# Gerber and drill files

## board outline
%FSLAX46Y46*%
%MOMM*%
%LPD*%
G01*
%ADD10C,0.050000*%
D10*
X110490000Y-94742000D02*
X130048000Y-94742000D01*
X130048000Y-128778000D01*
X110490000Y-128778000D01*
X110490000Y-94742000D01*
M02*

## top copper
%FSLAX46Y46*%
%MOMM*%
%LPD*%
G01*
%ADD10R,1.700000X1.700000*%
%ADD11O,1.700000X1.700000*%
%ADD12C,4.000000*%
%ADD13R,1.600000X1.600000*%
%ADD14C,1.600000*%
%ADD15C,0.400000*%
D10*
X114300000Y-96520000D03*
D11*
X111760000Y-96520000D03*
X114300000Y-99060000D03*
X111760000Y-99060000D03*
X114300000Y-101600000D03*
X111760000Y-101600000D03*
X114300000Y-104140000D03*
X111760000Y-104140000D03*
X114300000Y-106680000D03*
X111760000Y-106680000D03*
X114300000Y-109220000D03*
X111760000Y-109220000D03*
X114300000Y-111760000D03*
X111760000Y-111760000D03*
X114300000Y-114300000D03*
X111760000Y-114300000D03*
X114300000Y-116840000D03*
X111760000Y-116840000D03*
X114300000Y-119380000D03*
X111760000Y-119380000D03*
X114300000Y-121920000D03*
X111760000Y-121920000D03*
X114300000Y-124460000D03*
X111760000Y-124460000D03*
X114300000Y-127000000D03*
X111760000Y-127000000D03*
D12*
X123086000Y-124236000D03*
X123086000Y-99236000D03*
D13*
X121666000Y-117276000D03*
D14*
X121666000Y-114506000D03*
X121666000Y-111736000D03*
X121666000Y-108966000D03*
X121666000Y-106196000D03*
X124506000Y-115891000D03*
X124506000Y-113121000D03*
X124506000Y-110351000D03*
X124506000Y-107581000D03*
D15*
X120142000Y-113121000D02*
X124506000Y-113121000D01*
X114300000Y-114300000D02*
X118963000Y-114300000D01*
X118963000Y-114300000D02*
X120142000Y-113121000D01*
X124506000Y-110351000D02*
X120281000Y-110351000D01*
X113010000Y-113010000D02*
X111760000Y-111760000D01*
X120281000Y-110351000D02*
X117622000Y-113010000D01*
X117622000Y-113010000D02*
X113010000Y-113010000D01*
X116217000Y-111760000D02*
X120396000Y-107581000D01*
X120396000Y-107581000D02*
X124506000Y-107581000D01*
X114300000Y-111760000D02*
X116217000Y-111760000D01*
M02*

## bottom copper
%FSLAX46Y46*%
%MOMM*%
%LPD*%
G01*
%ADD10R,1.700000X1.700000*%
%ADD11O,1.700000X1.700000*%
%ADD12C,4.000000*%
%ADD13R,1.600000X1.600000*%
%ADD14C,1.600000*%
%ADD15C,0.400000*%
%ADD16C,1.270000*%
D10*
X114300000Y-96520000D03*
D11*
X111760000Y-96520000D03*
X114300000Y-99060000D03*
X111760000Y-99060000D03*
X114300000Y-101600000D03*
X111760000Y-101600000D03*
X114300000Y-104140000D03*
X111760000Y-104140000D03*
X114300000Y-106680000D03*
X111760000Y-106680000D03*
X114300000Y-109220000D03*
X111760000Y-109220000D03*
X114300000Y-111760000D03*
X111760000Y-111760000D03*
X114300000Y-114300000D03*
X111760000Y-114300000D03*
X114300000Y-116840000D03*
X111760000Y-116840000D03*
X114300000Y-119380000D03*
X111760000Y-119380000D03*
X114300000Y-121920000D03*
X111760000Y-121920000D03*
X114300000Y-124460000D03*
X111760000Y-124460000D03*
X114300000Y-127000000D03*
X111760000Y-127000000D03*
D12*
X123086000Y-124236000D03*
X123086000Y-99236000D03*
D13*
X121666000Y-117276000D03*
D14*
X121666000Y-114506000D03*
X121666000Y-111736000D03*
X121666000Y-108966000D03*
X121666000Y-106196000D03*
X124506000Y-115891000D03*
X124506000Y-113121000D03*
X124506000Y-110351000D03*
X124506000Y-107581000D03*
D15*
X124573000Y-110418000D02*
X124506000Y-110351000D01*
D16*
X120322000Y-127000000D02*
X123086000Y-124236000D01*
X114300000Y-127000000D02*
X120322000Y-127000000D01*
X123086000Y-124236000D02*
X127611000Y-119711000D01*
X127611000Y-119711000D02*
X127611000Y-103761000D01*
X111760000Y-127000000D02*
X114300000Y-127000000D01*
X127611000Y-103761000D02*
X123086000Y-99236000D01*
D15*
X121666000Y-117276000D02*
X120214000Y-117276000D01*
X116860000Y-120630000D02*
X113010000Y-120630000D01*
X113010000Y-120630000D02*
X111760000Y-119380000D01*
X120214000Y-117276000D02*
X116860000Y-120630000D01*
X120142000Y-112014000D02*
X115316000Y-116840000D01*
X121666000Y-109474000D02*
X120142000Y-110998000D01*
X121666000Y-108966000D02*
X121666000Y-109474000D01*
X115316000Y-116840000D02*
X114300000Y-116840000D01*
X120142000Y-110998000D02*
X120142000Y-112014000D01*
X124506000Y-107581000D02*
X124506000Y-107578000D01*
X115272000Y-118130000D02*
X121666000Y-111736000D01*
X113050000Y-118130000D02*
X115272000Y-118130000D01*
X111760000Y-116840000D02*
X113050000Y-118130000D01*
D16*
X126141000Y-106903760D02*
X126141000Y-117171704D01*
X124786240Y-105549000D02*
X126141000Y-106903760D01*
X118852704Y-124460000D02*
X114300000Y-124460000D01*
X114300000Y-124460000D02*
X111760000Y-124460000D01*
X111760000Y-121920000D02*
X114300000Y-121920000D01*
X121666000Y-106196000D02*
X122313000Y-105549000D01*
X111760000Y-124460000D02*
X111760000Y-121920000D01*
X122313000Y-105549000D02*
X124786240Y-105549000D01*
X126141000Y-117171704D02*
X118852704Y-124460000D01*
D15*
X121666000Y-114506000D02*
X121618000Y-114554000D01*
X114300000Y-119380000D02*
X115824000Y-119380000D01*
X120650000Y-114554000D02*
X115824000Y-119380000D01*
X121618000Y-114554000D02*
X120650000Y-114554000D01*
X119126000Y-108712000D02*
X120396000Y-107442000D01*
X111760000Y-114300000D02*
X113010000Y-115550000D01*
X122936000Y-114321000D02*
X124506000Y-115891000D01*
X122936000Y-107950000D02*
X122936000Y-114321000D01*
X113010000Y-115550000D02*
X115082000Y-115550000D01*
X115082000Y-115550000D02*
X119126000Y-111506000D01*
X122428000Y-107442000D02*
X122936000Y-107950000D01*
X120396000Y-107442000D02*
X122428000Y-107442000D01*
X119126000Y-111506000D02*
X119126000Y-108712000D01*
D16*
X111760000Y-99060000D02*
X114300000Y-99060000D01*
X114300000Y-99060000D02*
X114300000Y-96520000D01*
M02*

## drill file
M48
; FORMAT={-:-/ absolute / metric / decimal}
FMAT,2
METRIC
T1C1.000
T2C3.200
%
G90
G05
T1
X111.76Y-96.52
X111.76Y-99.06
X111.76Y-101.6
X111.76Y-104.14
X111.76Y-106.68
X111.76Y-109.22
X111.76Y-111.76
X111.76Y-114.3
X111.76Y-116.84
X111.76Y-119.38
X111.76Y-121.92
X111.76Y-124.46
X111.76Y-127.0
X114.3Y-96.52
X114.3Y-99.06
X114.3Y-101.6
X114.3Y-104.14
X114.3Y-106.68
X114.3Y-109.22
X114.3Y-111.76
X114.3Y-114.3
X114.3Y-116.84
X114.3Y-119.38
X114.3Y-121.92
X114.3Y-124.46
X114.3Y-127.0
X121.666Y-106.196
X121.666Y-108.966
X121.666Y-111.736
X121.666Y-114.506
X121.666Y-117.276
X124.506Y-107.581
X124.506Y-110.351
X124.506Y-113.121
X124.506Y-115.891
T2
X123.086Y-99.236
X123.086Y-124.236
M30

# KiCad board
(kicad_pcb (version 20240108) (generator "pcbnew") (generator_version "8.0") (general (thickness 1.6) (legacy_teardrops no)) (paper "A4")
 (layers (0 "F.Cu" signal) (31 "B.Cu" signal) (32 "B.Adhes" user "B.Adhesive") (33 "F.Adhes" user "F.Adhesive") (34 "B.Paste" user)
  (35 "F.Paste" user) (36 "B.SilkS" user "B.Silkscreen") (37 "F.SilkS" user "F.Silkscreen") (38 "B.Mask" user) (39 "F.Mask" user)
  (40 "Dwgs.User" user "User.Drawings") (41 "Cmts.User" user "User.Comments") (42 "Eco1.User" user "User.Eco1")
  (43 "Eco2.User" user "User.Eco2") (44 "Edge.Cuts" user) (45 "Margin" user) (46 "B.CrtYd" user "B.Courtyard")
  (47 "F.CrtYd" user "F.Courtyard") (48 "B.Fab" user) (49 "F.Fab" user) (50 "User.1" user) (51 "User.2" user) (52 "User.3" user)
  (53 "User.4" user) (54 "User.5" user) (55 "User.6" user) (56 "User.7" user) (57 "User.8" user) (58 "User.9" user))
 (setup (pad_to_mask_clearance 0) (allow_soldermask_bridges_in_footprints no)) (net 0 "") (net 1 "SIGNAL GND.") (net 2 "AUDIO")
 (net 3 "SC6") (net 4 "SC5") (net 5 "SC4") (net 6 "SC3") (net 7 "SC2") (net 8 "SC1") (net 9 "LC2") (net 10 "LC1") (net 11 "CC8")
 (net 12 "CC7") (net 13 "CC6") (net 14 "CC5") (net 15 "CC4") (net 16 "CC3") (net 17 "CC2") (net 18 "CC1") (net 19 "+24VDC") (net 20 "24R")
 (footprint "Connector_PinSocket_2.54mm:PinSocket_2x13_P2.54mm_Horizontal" (layer "F.Cu") (at 114.3 96.52)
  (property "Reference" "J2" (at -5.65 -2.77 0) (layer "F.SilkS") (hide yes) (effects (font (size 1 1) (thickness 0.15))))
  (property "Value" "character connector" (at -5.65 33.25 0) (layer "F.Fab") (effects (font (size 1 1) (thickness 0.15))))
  (pad "1" thru_hole rect (at 0 0) (size 1.7 1.7) (drill 1) (layers "*.Cu" "*.Mask") (remove_unused_layers no) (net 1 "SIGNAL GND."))
  (pad "2" thru_hole oval (at -2.54 0) (size 1.7 1.7) (drill 1) (layers "*.Cu" "*.Mask") (remove_unused_layers no) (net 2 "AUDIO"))
  (pad "3" thru_hole oval (at 0 2.54) (size 1.7 1.7) (drill 1) (layers "*.Cu" "*.Mask") (remove_unused_layers no) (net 1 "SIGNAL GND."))
  (pad "4" thru_hole oval (at -2.54 2.54) (size 1.7 1.7) (drill 1) (layers "*.Cu" "*.Mask") (remove_unused_layers no) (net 1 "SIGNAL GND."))
  (pad "5" thru_hole oval (at 0 5.08) (size 1.7 1.7) (drill 1) (layers "*.Cu" "*.Mask") (remove_unused_layers no) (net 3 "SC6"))
  (pad "6" thru_hole oval (at -2.54 5.08) (size 1.7 1.7) (drill 1) (layers "*.Cu" "*.Mask") (remove_unused_layers no) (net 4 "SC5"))
  (pad "7" thru_hole oval (at 0 7.62) (size 1.7 1.7) (drill 1) (layers "*.Cu" "*.Mask") (remove_unused_layers no) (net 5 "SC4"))
  (pad "8" thru_hole oval (at -2.54 7.62) (size 1.7 1.7) (drill 1) (layers "*.Cu" "*.Mask") (remove_unused_layers no) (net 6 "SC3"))
  (pad "9" thru_hole oval (at 0 10.16) (size 1.7 1.7) (drill 1) (layers "*.Cu" "*.Mask") (remove_unused_layers no) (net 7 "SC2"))
  (pad "10" thru_hole oval (at -2.54 10.16) (size 1.7 1.7) (drill 1) (layers "*.Cu" "*.Mask") (remove_unused_layers no) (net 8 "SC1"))
  (pad "11" thru_hole oval (at 0 12.7) (size 1.7 1.7) (drill 1) (layers "*.Cu" "*.Mask") (remove_unused_layers no) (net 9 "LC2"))
  (pad "12" thru_hole oval (at -2.54 12.7) (size 1.7 1.7) (drill 1) (layers "*.Cu" "*.Mask") (remove_unused_layers no) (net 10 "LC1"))
  (pad "13" thru_hole oval (at 0 15.24) (size 1.7 1.7) (drill 1) (layers "*.Cu" "*.Mask") (remove_unused_layers no) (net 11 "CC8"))
  (pad "14" thru_hole oval (at -2.54 15.24) (size 1.7 1.7) (drill 1) (layers "*.Cu" "*.Mask") (remove_unused_layers no) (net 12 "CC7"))
  (pad "15" thru_hole oval (at 0 17.78) (size 1.7 1.7) (drill 1) (layers "*.Cu" "*.Mask") (remove_unused_layers no) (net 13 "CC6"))
  (pad "16" thru_hole oval (at -2.54 17.78) (size 1.7 1.7) (drill 1) (layers "*.Cu" "*.Mask") (remove_unused_layers no) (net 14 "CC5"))
  (pad "17" thru_hole oval (at 0 20.32) (size 1.7 1.7) (drill 1) (layers "*.Cu" "*.Mask") (remove_unused_layers no) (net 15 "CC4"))
  (pad "18" thru_hole oval (at -2.54 20.32) (size 1.7 1.7) (drill 1) (layers "*.Cu" "*.Mask") (remove_unused_layers no) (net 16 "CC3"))
  (pad "19" thru_hole oval (at 0 22.86) (size 1.7 1.7) (drill 1) (layers "*.Cu" "*.Mask") (remove_unused_layers no) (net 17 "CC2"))
  (pad "20" thru_hole oval (at -2.54 22.86) (size 1.7 1.7) (drill 1) (layers "*.Cu" "*.Mask") (remove_unused_layers no) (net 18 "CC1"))
  (pad "21" thru_hole oval (at 0 25.4) (size 1.7 1.7) (drill 1) (layers "*.Cu" "*.Mask") (remove_unused_layers no) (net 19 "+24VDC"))
  (pad "22" thru_hole oval (at -2.54 25.4) (size 1.7 1.7) (drill 1) (layers "*.Cu" "*.Mask") (remove_unused_layers no) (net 19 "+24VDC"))
  (pad "23" thru_hole oval (at 0 27.94) (size 1.7 1.7) (drill 1) (layers "*.Cu" "*.Mask") (remove_unused_layers no) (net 19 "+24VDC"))
  (pad "24" thru_hole oval (at -2.54 27.94) (size 1.7 1.7) (drill 1) (layers "*.Cu" "*.Mask") (remove_unused_layers no) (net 19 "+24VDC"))
  (pad "25" thru_hole oval (at 0 30.48) (size 1.7 1.7) (drill 1) (layers "*.Cu" "*.Mask") (remove_unused_layers no) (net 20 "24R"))
  (pad "26" thru_hole oval (at -2.54 30.48) (size 1.7 1.7) (drill 1) (layers "*.Cu" "*.Mask") (remove_unused_layers no) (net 20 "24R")))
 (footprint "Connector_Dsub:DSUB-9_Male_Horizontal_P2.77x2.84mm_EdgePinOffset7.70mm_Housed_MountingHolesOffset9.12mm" (layer "F.Cu")
  (at 121.666 117.276 90)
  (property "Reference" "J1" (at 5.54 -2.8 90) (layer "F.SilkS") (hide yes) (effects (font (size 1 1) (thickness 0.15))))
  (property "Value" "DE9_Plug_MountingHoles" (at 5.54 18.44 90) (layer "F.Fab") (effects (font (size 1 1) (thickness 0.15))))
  (pad "0" thru_hole circle (at -6.96 1.42 90) (size 4 4) (drill 3.2) (layers "*.Cu" "*.Mask") (remove_unused_layers no) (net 20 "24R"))
  (pad "0" thru_hole circle (at 18.04 1.42 90) (size 4 4) (drill 3.2) (layers "*.Cu" "*.Mask") (remove_unused_layers no) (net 20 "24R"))
  (pad "1" thru_hole rect (at 0 0 90) (size 1.6 1.6) (drill 1) (layers "*.Cu" "*.Mask") (remove_unused_layers no) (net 18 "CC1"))
  (pad "2" thru_hole circle (at 2.77 0 90) (size 1.6 1.6) (drill 1) (layers "*.Cu" "*.Mask") (remove_unused_layers no) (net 17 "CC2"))
  (pad "3" thru_hole circle (at 5.54 0 90) (size 1.6 1.6) (drill 1) (layers "*.Cu" "*.Mask") (remove_unused_layers no) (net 16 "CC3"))
  (pad "4" thru_hole circle (at 8.31 0 90) (size 1.6 1.6) (drill 1) (layers "*.Cu" "*.Mask") (remove_unused_layers no) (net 15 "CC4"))
  (pad "5" thru_hole circle (at 11.08 0 90) (size 1.6 1.6) (drill 1) (layers "*.Cu" "*.Mask") (remove_unused_layers no) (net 19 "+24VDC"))
  (pad "6" thru_hole circle (at 1.385 2.84 90) (size 1.6 1.6) (drill 1) (layers "*.Cu" "*.Mask") (remove_unused_layers no) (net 14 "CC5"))
  (pad "7" thru_hole circle (at 4.155 2.84 90) (size 1.6 1.6) (drill 1) (layers "*.Cu" "*.Mask") (remove_unused_layers no) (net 13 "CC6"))
  (pad "8" thru_hole circle (at 6.925 2.84 90) (size 1.6 1.6) (drill 1) (layers "*.Cu" "*.Mask") (remove_unused_layers no) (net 12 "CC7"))
  (pad "9" thru_hole circle (at 9.695 2.84 90) (size 1.6 1.6) (drill 1) (layers "*.Cu" "*.Mask") (remove_unused_layers no) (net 11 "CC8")))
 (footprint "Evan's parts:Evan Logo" (layer "B.Cu") (at 127.508 97.536 -90)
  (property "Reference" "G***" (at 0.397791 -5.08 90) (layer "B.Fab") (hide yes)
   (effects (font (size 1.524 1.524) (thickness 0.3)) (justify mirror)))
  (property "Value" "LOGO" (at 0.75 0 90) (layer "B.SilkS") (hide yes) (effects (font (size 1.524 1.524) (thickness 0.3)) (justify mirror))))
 (gr_rect (start 110.49 94.742) (end 130.048 128.778) (stroke (width 0.05) (type default)) (fill none) (layer "Edge.Cuts"))
 (segment (start 120.142 113.121) (end 124.506 113.121) (width 0.4) (layer "F.Cu") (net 13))
 (segment (start 114.3 114.3) (end 118.963 114.3) (width 0.4) (layer "F.Cu") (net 13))
 (segment (start 118.963 114.3) (end 120.142 113.121) (width 0.4) (layer "F.Cu") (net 13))
 (segment (start 124.506 110.351) (end 120.281 110.351) (width 0.4) (layer "F.Cu") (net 12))
 (segment (start 113.01 113.01) (end 111.76 111.76) (width 0.4) (layer "F.Cu") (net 12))
 (segment (start 120.281 110.351) (end 117.622 113.01) (width 0.4) (layer "F.Cu") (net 12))
 (segment (start 117.622 113.01) (end 113.01 113.01) (width 0.4) (layer "F.Cu") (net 12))
 (segment (start 124.573 110.418) (end 124.506 110.351) (width 0.4) (layer "B.Cu") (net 12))
 (segment (start 120.322 127) (end 123.086 124.236) (width 1.27) (layer "B.Cu") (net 20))
 (segment (start 114.3 127) (end 120.322 127) (width 1.27) (layer "B.Cu") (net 20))
 (segment (start 123.086 124.236) (end 127.611 119.711) (width 1.27) (layer "B.Cu") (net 20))
 (segment (start 127.611 119.711) (end 127.611 103.761) (width 1.27) (layer "B.Cu") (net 20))
 (segment (start 111.76 127) (end 114.3 127) (width 1.27) (layer "B.Cu") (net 20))
 (segment (start 127.611 103.761) (end 123.086 99.236) (width 1.27) (layer "B.Cu") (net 20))
 (segment (start 121.666 117.276) (end 120.214 117.276) (width 0.4) (layer "B.Cu") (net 18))
 (segment (start 116.86 120.63) (end 113.01 120.63) (width 0.4) (layer "B.Cu") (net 18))
 (segment (start 113.01 120.63) (end 111.76 119.38) (width 0.4) (layer "B.Cu") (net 18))
 (segment (start 120.214 117.276) (end 116.86 120.63) (width 0.4) (layer "B.Cu") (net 18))
 (segment (start 120.142 112.014) (end 115.316 116.84) (width 0.4) (layer "B.Cu") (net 15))
 (segment (start 121.666 109.474) (end 120.142 110.998) (width 0.4) (layer "B.Cu") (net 15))
 (segment (start 121.666 108.966) (end 121.666 109.474) (width 0.4) (layer "B.Cu") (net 15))
 (segment (start 115.316 116.84) (end 114.3 116.84) (width 0.4) (layer "B.Cu") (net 15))
 (segment (start 120.142 110.998) (end 120.142 112.014) (width 0.4) (layer "B.Cu") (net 15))
 (segment (start 116.217 111.76) (end 120.396 107.581) (width 0.4) (layer "F.Cu") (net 11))
 (segment (start 120.396 107.581) (end 124.506 107.581) (width 0.4) (layer "F.Cu") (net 11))
 (segment (start 114.3 111.76) (end 116.217 111.76) (width 0.4) (layer "F.Cu") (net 11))
 (segment (start 124.506 107.581) (end 124.506 107.578) (width 0.4) (layer "B.Cu") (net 11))
 (segment (start 115.272 118.13) (end 121.666 111.736) (width 0.4) (layer "B.Cu") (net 16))
 (segment (start 113.05 118.13) (end 115.272 118.13) (width 0.4) (layer "B.Cu") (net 16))
 (segment (start 111.76 116.84) (end 113.05 118.13) (width 0.4) (layer "B.Cu") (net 16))
 (segment (start 126.141 106.90376) (end 126.141 117.171704) (width 1.27) (layer "B.Cu") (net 19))
 (segment (start 124.78624 105.549) (end 126.141 106.90376) (width 1.27) (layer "B.Cu") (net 19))
 (segment (start 118.852704 124.46) (end 114.3 124.46) (width 1.27) (layer "B.Cu") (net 19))
 (segment (start 114.3 124.46) (end 111.76 124.46) (width 1.27) (layer "B.Cu") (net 19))
 (segment (start 111.76 121.92) (end 114.3 121.92) (width 1.27) (layer "B.Cu") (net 19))
 (segment (start 121.666 106.196) (end 122.313 105.549) (width 1.27) (layer "B.Cu") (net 19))
 (segment (start 111.76 124.46) (end 111.76 121.92) (width 1.27) (layer "B.Cu") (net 19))
 (segment (start 122.313 105.549) (end 124.78624 105.549) (width 1.27) (layer "B.Cu") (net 19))
 (segment (start 126.141 117.171704) (end 118.852704 124.46) (width 1.27) (layer "B.Cu") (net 19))
 (segment (start 121.666 114.506) (end 121.618 114.554) (width 0.4) (layer "B.Cu") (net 17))
 (segment (start 114.3 119.38) (end 115.824 119.38) (width 0.4) (layer "B.Cu") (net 17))
 (segment (start 120.65 114.554) (end 115.824 119.38) (width 0.4) (layer "B.Cu") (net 17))
 (segment (start 121.618 114.554) (end 120.65 114.554) (width 0.4) (layer "B.Cu") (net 17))
 (segment (start 119.126 108.712) (end 120.396 107.442) (width 0.4) (layer "B.Cu") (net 14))
 (segment (start 111.76 114.3) (end 113.01 115.55) (width 0.4) (layer "B.Cu") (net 14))
 (segment (start 122.936 114.321) (end 124.506 115.891) (width 0.4) (layer "B.Cu") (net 14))
 (segment (start 122.936 107.95) (end 122.936 114.321) (width 0.4) (layer "B.Cu") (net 14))
 (segment (start 113.01 115.55) (end 115.082 115.55) (width 0.4) (layer "B.Cu") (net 14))
 (segment (start 115.082 115.55) (end 119.126 111.506) (width 0.4) (layer "B.Cu") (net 14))
 (segment (start 122.428 107.442) (end 122.936 107.95) (width 0.4) (layer "B.Cu") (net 14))
 (segment (start 120.396 107.442) (end 122.428 107.442) (width 0.4) (layer "B.Cu") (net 14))
 (segment (start 119.126 111.506) (end 119.126 108.712) (width 0.4) (layer "B.Cu") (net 14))
 (segment (start 111.76 99.06) (end 114.3 99.06) (width 1.27) (layer "B.Cu") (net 1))
 (segment (start 114.3 99.06) (end 114.3 96.52) (width 1.27) (layer "B.Cu") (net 1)))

